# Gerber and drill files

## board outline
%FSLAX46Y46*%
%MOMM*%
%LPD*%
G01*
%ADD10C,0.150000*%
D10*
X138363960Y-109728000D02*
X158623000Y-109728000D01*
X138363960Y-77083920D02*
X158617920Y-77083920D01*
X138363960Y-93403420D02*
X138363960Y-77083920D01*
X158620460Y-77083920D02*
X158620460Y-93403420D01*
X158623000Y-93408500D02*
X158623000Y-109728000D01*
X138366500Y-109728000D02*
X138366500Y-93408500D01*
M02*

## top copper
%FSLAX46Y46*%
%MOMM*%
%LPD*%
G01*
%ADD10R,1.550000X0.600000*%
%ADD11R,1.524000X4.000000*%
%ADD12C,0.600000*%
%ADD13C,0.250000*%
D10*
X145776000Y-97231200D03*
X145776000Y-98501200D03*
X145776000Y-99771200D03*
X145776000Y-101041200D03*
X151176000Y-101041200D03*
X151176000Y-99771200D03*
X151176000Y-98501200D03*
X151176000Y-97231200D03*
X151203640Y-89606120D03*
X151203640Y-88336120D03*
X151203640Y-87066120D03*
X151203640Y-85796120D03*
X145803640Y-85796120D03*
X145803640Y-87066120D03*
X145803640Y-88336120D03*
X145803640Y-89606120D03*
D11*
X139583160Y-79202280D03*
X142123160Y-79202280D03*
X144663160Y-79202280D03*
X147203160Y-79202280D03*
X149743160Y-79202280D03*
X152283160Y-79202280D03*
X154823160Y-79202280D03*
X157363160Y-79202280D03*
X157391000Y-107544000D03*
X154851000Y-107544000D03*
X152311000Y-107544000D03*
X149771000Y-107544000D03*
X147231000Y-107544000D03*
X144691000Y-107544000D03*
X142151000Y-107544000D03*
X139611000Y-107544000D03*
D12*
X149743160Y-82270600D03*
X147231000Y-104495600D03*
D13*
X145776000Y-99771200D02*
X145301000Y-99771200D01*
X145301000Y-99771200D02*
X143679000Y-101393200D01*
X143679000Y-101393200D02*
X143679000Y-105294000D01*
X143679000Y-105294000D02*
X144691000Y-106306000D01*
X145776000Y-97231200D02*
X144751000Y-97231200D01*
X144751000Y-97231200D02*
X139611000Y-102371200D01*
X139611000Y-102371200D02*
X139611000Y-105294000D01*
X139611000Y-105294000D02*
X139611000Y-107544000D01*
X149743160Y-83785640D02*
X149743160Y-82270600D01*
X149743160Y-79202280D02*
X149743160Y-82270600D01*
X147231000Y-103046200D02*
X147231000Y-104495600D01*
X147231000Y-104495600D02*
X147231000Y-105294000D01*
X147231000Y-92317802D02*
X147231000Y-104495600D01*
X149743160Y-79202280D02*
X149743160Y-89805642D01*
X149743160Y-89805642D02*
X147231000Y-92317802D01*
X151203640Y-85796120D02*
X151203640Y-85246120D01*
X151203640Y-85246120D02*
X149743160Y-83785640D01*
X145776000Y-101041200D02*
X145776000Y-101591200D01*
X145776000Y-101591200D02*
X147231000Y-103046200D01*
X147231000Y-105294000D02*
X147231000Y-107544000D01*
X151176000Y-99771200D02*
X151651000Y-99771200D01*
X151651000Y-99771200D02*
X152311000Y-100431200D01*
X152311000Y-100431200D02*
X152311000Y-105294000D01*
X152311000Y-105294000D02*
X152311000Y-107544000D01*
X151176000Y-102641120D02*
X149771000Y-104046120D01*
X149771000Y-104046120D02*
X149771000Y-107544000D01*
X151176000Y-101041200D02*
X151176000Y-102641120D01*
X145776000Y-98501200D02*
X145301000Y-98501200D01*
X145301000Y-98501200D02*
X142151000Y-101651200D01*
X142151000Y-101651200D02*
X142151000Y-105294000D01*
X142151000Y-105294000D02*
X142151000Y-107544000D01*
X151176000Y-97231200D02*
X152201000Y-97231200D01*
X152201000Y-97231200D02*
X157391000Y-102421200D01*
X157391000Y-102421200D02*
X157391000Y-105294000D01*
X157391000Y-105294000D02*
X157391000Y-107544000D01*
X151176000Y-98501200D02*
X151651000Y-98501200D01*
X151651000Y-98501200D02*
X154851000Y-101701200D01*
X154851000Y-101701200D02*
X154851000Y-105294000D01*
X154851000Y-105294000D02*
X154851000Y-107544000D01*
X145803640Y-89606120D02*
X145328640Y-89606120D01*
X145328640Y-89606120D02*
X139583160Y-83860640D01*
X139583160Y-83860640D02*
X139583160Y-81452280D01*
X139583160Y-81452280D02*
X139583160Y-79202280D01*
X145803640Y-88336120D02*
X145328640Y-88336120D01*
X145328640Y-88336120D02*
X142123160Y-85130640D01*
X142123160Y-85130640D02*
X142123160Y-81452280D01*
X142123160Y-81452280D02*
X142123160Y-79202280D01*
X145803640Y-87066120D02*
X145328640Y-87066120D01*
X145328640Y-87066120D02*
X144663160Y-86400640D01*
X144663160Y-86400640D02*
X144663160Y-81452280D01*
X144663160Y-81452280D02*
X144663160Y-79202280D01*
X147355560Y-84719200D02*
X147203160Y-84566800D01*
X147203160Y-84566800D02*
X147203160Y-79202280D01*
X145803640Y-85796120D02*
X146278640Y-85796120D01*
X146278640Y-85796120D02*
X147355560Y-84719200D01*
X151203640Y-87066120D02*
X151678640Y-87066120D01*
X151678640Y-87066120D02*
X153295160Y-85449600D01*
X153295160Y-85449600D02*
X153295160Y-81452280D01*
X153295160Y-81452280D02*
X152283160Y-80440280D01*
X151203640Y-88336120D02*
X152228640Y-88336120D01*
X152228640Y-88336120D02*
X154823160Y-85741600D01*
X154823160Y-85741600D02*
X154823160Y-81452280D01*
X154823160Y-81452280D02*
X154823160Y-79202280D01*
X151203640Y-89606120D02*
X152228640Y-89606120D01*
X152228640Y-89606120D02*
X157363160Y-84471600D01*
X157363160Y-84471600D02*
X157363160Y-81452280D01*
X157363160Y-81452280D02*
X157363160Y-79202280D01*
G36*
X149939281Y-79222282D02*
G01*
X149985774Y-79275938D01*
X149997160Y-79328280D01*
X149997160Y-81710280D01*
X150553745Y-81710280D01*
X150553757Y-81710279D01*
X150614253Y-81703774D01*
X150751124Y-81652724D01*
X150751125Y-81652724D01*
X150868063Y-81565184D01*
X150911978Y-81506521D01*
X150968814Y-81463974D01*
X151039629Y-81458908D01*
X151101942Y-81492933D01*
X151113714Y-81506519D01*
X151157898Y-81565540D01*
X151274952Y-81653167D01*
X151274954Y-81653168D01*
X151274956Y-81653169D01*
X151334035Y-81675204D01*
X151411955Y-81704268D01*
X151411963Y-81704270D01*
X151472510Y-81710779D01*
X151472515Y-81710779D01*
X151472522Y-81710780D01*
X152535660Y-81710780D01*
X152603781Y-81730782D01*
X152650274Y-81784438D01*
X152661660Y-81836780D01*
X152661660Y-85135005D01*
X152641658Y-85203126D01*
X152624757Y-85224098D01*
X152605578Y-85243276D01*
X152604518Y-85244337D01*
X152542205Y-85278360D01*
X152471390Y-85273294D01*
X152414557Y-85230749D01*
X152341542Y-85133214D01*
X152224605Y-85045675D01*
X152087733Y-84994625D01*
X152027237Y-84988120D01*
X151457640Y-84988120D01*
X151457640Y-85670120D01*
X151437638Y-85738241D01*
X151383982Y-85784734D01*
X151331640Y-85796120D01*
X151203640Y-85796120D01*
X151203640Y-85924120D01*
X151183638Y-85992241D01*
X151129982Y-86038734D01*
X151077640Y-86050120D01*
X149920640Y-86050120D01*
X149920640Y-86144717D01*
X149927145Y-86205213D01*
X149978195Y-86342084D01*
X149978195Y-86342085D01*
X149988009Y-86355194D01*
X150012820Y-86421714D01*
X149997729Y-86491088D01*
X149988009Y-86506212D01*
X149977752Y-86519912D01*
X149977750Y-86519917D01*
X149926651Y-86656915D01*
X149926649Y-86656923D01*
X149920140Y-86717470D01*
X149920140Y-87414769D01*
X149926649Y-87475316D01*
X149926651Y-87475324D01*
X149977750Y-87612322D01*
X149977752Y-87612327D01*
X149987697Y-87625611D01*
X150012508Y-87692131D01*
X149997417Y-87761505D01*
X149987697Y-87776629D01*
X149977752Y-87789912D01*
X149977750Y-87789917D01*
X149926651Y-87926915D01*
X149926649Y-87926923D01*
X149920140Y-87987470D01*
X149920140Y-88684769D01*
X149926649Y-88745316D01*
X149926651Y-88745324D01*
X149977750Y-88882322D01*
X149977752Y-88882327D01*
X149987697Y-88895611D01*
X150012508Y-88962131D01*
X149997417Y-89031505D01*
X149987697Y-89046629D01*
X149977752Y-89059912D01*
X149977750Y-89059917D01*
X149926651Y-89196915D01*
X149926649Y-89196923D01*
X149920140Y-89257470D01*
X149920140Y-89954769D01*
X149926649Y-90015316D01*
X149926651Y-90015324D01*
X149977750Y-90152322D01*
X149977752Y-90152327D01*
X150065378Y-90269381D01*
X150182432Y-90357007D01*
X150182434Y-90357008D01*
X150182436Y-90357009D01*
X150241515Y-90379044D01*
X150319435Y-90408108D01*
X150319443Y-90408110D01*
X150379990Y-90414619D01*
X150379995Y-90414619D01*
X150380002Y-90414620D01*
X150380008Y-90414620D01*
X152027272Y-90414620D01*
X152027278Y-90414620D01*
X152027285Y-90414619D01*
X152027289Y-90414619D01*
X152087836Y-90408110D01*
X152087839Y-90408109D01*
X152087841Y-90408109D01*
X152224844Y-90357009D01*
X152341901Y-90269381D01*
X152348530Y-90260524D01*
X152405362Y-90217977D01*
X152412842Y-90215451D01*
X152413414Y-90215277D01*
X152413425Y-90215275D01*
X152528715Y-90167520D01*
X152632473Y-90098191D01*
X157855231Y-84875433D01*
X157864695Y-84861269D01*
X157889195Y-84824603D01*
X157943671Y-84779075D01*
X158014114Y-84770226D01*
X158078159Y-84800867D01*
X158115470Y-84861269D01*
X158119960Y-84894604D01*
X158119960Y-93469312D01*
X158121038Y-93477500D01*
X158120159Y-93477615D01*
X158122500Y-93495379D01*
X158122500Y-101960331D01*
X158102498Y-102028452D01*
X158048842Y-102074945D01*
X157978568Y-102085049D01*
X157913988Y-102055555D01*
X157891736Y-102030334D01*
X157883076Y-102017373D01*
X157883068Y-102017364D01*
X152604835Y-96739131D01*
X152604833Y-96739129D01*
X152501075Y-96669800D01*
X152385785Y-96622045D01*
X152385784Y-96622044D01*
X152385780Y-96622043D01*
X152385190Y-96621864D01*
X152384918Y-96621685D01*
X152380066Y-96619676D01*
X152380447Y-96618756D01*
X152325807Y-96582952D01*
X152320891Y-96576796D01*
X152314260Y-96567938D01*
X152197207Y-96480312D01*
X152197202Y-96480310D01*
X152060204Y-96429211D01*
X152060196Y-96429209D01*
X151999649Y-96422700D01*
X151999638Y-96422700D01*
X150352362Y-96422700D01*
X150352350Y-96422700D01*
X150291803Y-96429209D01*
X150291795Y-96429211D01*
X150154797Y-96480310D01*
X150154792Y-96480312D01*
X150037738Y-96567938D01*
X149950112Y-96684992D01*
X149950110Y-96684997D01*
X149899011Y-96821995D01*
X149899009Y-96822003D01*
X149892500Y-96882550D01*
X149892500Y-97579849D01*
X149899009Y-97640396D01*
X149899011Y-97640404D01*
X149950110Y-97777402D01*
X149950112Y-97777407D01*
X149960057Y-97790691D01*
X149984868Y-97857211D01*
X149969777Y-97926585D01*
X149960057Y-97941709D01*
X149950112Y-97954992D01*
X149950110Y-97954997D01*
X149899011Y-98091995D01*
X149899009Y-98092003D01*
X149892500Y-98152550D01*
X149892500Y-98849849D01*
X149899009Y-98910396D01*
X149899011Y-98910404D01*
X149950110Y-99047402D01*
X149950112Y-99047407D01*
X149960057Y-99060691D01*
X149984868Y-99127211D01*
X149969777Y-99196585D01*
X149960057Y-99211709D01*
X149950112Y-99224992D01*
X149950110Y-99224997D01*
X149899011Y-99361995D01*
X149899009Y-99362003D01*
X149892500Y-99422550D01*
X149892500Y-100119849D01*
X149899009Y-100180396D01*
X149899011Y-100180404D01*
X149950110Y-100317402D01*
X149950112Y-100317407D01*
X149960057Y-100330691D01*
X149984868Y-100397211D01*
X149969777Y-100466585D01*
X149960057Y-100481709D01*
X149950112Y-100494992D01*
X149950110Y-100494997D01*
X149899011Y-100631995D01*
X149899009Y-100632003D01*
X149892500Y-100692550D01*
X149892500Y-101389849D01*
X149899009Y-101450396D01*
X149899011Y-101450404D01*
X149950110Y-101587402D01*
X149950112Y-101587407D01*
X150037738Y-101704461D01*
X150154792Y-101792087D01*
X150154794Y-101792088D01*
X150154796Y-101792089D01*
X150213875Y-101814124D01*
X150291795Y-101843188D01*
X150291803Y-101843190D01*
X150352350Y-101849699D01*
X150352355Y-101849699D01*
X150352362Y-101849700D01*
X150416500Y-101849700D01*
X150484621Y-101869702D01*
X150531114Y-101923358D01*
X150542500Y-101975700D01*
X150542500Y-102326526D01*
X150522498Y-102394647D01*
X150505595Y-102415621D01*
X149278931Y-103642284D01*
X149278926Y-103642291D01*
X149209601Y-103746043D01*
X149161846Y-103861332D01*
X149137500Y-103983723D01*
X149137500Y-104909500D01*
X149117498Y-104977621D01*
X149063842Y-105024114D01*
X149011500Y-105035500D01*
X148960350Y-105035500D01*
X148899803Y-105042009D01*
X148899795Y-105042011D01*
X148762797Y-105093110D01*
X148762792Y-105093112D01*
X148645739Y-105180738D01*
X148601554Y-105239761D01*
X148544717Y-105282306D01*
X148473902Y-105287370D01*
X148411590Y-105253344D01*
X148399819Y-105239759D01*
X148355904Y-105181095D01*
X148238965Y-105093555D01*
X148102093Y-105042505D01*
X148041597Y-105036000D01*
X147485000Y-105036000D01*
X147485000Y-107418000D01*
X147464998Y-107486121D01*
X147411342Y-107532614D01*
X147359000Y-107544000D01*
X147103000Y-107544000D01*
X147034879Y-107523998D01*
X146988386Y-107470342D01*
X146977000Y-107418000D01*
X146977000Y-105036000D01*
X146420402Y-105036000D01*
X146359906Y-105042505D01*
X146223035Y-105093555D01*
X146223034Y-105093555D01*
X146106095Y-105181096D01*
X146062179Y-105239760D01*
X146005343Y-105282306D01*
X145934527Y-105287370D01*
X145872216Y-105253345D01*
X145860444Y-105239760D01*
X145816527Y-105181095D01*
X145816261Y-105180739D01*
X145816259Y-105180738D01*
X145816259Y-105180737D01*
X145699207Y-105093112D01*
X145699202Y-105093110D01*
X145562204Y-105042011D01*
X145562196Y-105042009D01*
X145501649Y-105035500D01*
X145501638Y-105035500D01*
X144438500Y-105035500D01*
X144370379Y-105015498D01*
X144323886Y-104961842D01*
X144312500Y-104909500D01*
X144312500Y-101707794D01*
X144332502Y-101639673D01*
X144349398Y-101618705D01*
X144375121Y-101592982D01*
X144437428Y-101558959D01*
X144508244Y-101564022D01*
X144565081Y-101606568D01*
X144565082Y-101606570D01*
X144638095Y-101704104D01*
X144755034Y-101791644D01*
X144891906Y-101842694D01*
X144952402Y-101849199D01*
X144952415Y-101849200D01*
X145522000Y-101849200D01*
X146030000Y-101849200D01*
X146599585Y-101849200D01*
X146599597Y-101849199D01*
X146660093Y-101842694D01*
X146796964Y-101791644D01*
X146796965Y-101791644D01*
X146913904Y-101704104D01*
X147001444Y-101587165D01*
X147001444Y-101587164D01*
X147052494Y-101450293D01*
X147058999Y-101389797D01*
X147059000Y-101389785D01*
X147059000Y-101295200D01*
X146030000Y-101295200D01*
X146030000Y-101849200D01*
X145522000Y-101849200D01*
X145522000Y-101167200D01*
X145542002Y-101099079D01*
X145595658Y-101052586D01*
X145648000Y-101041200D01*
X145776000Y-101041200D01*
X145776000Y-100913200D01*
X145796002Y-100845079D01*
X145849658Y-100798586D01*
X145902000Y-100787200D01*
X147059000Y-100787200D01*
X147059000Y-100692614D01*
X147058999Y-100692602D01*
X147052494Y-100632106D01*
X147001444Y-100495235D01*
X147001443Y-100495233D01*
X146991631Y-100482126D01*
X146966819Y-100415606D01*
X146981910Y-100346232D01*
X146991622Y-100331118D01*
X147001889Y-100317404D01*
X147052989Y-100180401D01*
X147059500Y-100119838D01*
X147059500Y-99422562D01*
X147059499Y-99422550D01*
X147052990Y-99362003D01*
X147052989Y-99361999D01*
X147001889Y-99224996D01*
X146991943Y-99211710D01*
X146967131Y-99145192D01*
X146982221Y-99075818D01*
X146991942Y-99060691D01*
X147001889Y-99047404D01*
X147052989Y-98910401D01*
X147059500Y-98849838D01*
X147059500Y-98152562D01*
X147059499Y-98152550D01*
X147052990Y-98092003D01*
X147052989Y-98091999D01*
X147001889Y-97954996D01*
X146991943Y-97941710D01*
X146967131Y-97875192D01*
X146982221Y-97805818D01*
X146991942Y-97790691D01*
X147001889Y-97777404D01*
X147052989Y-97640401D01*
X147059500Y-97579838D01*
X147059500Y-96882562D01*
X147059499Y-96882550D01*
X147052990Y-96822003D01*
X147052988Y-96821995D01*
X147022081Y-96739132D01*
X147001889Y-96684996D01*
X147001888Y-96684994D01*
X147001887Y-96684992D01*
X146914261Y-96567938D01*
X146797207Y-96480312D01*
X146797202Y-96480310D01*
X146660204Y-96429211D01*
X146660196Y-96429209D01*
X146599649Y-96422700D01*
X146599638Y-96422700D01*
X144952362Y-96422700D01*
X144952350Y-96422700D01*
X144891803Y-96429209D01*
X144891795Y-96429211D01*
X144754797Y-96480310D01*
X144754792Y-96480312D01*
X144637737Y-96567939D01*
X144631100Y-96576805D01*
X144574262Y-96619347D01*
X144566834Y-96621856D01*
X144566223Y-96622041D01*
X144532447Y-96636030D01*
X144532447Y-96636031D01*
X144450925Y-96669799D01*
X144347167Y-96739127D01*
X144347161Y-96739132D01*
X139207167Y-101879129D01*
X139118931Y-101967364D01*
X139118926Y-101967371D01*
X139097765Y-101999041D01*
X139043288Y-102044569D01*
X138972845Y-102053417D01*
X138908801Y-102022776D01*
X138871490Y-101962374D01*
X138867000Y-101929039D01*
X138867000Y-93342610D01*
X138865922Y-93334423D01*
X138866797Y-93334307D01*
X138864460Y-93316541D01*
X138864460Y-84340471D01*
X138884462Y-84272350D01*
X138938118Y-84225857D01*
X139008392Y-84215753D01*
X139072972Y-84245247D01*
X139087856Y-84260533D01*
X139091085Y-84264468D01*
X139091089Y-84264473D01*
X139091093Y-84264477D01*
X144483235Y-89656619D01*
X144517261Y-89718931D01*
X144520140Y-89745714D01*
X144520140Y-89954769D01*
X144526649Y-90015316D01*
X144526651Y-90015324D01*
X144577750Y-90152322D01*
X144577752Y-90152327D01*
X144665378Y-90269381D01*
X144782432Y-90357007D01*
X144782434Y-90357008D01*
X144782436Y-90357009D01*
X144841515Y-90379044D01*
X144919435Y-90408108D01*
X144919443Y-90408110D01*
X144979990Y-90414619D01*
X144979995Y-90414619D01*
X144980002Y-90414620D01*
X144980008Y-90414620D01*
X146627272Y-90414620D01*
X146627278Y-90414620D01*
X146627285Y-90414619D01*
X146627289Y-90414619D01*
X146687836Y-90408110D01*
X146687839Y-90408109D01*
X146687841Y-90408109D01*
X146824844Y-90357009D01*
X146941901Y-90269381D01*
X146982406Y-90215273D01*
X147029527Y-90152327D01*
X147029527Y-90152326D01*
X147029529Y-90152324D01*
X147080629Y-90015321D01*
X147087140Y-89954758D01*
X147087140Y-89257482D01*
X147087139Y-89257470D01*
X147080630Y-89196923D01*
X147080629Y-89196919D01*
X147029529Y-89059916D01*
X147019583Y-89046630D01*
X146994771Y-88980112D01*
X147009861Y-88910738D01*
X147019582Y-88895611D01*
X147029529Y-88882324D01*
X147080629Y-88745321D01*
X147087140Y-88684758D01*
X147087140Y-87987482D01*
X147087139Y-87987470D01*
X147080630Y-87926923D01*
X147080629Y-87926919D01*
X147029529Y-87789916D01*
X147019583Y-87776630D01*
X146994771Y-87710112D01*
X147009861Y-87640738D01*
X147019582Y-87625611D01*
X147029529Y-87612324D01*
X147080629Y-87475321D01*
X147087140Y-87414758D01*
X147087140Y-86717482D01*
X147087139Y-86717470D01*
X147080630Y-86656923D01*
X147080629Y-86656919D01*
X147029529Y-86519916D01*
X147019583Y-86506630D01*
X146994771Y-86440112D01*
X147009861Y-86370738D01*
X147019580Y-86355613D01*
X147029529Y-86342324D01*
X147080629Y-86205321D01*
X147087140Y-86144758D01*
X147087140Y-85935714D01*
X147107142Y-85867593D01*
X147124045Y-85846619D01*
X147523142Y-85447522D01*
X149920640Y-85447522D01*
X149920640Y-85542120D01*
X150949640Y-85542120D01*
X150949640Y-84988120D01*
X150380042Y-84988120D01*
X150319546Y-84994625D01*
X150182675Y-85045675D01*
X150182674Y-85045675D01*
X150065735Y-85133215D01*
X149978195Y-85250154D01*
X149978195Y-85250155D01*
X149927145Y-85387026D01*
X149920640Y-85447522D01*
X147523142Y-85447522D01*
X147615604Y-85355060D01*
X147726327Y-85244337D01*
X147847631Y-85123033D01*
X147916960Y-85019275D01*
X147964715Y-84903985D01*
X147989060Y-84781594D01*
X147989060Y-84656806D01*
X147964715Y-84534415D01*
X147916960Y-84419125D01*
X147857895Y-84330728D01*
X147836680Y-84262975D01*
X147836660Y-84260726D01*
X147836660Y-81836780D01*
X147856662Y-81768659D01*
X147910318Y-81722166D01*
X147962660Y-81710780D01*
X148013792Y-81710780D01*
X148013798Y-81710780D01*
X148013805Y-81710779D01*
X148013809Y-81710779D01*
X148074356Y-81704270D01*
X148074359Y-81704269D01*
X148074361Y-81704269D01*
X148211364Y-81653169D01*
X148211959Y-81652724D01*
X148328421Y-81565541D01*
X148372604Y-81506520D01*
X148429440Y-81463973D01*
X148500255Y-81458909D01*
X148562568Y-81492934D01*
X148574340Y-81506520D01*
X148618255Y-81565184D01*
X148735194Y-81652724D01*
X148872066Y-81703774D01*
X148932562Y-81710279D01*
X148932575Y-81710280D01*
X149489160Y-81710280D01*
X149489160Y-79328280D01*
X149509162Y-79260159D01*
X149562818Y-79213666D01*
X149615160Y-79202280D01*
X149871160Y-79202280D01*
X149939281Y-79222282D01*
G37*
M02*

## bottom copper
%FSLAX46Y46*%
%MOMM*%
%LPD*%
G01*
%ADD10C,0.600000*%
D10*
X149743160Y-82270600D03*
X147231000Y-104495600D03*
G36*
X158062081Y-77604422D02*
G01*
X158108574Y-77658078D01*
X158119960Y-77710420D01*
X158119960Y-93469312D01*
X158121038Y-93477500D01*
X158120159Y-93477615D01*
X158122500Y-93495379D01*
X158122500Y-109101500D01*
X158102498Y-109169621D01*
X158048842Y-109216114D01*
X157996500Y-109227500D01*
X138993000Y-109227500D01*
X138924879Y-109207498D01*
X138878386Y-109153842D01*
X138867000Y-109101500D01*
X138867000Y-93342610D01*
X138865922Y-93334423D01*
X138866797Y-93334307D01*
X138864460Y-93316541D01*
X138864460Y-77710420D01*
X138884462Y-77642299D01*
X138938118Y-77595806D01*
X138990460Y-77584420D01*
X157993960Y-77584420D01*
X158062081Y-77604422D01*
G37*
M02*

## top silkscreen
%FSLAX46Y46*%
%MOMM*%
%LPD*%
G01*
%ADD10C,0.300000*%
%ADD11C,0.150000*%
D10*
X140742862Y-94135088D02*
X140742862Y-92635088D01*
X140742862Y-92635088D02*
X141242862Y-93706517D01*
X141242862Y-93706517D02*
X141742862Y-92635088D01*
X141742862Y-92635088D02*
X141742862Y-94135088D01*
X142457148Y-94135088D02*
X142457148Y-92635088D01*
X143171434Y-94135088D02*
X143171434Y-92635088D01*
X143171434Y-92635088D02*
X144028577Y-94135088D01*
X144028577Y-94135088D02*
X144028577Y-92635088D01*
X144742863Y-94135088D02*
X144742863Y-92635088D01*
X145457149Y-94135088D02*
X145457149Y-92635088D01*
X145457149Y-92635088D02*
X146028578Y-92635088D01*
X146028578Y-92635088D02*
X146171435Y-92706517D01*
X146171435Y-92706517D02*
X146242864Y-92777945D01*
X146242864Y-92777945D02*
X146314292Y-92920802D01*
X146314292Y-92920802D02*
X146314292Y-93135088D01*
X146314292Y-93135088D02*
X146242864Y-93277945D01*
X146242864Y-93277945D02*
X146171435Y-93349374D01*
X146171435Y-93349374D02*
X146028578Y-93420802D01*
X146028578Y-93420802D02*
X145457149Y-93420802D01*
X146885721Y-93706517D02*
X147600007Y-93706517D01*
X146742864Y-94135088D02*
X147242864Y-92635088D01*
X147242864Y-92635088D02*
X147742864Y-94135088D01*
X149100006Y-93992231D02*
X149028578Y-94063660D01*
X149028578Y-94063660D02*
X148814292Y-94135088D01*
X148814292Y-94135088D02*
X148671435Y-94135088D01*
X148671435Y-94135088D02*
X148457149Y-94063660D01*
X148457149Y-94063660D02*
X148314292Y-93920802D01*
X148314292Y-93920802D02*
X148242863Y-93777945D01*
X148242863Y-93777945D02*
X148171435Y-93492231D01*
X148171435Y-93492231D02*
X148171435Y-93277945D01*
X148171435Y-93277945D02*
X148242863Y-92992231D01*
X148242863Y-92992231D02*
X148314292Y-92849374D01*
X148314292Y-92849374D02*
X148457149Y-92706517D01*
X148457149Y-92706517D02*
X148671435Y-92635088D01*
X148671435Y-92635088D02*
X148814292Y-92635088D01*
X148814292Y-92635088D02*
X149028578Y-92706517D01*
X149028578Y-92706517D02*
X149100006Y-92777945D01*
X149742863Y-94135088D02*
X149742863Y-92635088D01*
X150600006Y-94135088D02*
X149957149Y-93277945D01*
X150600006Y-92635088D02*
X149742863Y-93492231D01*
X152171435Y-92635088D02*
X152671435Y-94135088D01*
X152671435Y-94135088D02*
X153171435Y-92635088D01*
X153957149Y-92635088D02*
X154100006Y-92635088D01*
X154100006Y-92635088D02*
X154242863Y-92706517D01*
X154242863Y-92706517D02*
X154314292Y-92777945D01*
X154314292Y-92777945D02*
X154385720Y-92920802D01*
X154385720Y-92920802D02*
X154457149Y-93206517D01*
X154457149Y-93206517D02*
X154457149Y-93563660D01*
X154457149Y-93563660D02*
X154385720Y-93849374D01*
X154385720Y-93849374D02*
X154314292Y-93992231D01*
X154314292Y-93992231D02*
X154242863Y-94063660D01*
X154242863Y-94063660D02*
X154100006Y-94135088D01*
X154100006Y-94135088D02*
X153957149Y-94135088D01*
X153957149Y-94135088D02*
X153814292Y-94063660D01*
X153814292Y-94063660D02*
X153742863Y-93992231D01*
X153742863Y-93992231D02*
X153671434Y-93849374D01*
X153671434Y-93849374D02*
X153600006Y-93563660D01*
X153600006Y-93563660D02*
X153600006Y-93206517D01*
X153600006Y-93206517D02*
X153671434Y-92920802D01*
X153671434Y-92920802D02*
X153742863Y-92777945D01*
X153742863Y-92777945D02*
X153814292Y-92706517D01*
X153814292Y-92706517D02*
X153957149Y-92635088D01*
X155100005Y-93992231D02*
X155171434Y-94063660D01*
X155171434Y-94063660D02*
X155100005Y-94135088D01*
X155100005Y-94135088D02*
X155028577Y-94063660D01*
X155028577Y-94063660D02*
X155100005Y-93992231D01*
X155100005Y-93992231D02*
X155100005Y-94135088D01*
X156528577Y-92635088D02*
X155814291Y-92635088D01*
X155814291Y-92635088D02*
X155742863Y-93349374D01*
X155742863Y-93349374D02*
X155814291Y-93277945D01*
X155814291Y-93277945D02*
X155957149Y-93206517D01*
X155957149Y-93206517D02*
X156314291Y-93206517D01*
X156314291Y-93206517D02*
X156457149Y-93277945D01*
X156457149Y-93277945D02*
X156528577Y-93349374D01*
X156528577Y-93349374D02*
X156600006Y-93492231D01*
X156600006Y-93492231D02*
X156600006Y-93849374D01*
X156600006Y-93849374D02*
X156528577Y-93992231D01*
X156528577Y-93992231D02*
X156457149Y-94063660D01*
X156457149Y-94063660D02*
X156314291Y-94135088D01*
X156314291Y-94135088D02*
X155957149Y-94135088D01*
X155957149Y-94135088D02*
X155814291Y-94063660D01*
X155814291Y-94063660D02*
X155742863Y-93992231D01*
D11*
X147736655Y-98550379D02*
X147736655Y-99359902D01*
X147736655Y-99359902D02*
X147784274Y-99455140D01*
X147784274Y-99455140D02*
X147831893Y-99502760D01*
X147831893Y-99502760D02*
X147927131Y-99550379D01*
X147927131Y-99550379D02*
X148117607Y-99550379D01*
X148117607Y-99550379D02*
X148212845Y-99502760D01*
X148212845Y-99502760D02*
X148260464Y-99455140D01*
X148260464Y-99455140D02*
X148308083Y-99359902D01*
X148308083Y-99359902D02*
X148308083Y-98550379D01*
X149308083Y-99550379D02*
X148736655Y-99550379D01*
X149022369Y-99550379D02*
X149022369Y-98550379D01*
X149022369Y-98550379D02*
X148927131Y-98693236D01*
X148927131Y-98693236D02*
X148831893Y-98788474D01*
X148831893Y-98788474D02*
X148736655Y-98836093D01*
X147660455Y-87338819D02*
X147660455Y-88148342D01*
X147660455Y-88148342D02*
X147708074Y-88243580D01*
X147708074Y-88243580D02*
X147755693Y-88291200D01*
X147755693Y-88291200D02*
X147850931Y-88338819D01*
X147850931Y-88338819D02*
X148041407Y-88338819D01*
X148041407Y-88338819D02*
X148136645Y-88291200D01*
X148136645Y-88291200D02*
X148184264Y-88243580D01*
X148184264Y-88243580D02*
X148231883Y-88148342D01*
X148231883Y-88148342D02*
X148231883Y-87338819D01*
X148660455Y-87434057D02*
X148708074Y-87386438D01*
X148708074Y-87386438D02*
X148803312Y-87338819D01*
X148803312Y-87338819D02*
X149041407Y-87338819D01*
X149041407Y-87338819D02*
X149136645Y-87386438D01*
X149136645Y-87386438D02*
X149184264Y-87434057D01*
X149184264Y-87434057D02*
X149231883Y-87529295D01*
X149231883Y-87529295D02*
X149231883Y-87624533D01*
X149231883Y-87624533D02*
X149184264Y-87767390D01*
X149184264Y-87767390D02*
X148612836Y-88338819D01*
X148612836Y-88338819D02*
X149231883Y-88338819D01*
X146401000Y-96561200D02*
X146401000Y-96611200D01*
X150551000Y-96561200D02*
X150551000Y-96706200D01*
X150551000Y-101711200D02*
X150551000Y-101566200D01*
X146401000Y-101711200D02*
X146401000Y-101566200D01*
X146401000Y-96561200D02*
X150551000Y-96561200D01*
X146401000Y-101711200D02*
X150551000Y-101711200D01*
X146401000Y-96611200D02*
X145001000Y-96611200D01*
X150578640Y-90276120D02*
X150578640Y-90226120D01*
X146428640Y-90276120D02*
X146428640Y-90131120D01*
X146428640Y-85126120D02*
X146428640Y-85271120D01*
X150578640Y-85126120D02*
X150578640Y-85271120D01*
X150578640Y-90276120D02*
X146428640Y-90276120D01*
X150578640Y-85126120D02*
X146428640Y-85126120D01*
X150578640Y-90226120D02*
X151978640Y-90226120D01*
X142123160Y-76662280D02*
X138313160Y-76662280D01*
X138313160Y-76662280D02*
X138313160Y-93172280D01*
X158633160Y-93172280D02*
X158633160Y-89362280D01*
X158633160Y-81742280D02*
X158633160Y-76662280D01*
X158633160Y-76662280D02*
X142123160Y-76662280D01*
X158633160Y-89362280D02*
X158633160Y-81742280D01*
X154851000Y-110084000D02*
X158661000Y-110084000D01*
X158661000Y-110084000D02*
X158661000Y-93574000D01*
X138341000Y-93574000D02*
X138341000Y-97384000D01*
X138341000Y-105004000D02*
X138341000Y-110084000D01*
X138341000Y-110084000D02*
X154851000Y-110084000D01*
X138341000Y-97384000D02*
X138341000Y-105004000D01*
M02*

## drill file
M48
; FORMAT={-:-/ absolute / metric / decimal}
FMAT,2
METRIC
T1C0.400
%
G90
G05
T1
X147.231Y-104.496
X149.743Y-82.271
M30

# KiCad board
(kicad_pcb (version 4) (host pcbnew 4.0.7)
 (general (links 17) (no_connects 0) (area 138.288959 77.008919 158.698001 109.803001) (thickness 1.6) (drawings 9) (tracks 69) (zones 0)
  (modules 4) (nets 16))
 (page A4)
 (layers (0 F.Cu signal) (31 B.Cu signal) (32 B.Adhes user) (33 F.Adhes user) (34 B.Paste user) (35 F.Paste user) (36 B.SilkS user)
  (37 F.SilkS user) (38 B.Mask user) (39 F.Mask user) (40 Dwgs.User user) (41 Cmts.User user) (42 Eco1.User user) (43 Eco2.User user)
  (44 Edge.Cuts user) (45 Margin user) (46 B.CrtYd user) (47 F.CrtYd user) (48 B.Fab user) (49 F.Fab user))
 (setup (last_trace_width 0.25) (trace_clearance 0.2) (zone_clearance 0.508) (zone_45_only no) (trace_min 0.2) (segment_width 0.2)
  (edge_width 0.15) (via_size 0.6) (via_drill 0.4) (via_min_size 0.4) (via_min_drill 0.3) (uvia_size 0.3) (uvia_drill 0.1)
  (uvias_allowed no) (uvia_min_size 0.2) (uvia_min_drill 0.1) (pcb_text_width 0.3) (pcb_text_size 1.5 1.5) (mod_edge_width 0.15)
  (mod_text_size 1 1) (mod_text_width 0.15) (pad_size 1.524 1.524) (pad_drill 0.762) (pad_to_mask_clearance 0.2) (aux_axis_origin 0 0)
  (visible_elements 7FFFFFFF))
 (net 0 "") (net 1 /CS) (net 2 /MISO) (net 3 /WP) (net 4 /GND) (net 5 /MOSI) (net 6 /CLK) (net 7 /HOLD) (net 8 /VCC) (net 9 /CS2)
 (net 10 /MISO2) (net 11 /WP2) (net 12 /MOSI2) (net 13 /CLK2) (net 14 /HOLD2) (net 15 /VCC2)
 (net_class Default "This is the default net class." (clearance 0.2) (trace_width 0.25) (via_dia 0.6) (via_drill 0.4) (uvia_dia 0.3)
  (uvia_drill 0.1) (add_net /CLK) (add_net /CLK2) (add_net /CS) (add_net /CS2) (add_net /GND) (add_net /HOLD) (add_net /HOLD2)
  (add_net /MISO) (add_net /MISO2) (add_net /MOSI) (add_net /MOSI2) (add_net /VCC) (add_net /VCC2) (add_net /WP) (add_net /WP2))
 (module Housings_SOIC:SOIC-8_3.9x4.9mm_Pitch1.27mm (layer F.Cu) (at 148.476 99.1362)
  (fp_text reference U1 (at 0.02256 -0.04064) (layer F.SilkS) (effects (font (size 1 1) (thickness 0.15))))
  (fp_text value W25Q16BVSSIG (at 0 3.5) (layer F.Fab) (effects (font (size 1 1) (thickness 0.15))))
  (fp_line (start -2.075 -2.575) (end -2.075 -2.525) (layer F.SilkS) (width 0.15))
  (fp_line (start 2.075 -2.575) (end 2.075 -2.43) (layer F.SilkS) (width 0.15))
  (fp_line (start 2.075 2.575) (end 2.075 2.43) (layer F.SilkS) (width 0.15))
  (fp_line (start -2.075 2.575) (end -2.075 2.43) (layer F.SilkS) (width 0.15))
  (fp_line (start -2.075 -2.575) (end 2.075 -2.575) (layer F.SilkS) (width 0.15))
  (fp_line (start -2.075 2.575) (end 2.075 2.575) (layer F.SilkS) (width 0.15))
  (fp_line (start -2.075 -2.525) (end -3.475 -2.525) (layer F.SilkS) (width 0.15))
  (pad 1 smd rect (at -2.7 -1.905) (size 1.55 0.6) (layers F.Cu F.Paste F.Mask) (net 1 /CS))
  (pad 2 smd rect (at -2.7 -0.635) (size 1.55 0.6) (layers F.Cu F.Paste F.Mask) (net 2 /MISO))
  (pad 3 smd rect (at -2.7 0.635) (size 1.55 0.6) (layers F.Cu F.Paste F.Mask) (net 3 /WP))
  (pad 4 smd rect (at -2.7 1.905) (size 1.55 0.6) (layers F.Cu F.Paste F.Mask) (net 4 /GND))
  (pad 5 smd rect (at 2.7 1.905) (size 1.55 0.6) (layers F.Cu F.Paste F.Mask) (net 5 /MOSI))
  (pad 6 smd rect (at 2.7 0.635) (size 1.55 0.6) (layers F.Cu F.Paste F.Mask) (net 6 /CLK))
  (pad 7 smd rect (at 2.7 -0.635) (size 1.55 0.6) (layers F.Cu F.Paste F.Mask) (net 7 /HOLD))
  (pad 8 smd rect (at 2.7 -1.905) (size 1.55 0.6) (layers F.Cu F.Paste F.Mask) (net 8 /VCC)))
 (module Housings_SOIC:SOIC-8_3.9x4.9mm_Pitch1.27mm (layer F.Cu) (at 148.50364 87.70112 180)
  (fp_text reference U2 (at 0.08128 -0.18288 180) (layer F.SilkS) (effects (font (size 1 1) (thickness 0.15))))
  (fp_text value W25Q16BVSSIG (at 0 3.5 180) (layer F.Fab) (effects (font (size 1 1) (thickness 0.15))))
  (fp_line (start -2.075 -2.575) (end -2.075 -2.525) (layer F.SilkS) (width 0.15))
  (fp_line (start 2.075 -2.575) (end 2.075 -2.43) (layer F.SilkS) (width 0.15))
  (fp_line (start 2.075 2.575) (end 2.075 2.43) (layer F.SilkS) (width 0.15))
  (fp_line (start -2.075 2.575) (end -2.075 2.43) (layer F.SilkS) (width 0.15))
  (fp_line (start -2.075 -2.575) (end 2.075 -2.575) (layer F.SilkS) (width 0.15))
  (fp_line (start -2.075 2.575) (end 2.075 2.575) (layer F.SilkS) (width 0.15))
  (fp_line (start -2.075 -2.525) (end -3.475 -2.525) (layer F.SilkS) (width 0.15))
  (pad 1 smd rect (at -2.7 -1.905 180) (size 1.55 0.6) (layers F.Cu F.Paste F.Mask) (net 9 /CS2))
  (pad 2 smd rect (at -2.7 -0.635 180) (size 1.55 0.6) (layers F.Cu F.Paste F.Mask) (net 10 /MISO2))
  (pad 3 smd rect (at -2.7 0.635 180) (size 1.55 0.6) (layers F.Cu F.Paste F.Mask) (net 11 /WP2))
  (pad 4 smd rect (at -2.7 1.905 180) (size 1.55 0.6) (layers F.Cu F.Paste F.Mask) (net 4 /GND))
  (pad 5 smd rect (at 2.7 1.905 180) (size 1.55 0.6) (layers F.Cu F.Paste F.Mask) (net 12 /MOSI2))
  (pad 6 smd rect (at 2.7 0.635 180) (size 1.55 0.6) (layers F.Cu F.Paste F.Mask) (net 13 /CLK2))
  (pad 7 smd rect (at 2.7 -0.635 180) (size 1.55 0.6) (layers F.Cu F.Paste F.Mask) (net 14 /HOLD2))
  (pad 8 smd rect (at 2.7 -1.905 180) (size 1.55 0.6) (layers F.Cu F.Paste F.Mask) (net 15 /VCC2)))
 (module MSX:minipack (layer F.Cu) (at 148.47316 81.74228 180)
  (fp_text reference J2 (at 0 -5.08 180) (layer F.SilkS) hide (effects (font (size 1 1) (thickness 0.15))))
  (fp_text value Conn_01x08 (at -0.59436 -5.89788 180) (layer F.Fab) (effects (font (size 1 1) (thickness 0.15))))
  (fp_line (start 6.35 5.08) (end 10.16 5.08) (layer F.SilkS) (width 0.15))
  (fp_line (start 10.16 5.08) (end 10.16 -11.43) (layer F.SilkS) (width 0.15))
  (fp_line (start -10.16 -11.43) (end -10.16 -7.62) (layer F.SilkS) (width 0.15))
  (fp_line (start -10.16 0) (end -10.16 5.08) (layer F.SilkS) (width 0.15))
  (fp_line (start -10.16 5.08) (end 6.35 5.08) (layer F.SilkS) (width 0.15))
  (fp_line (start -10.16 -7.62) (end -10.16 0) (layer F.SilkS) (width 0.15))
  (pad 8 smd rect (at 8.89 2.54 180) (size 1.524 4) (layers F.Cu F.Paste F.Mask) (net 15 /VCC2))
  (pad 7 smd rect (at 6.35 2.54 180) (size 1.524 4) (layers F.Cu F.Paste F.Mask) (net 14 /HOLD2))
  (pad 6 smd rect (at 3.81 2.54 180) (size 1.524 4) (layers F.Cu F.Paste F.Mask) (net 13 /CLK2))
  (pad 5 smd rect (at 1.27 2.54 180) (size 1.524 4) (layers F.Cu F.Paste F.Mask) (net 12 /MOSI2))
  (pad 4 smd rect (at -1.27 2.54 180) (size 1.524 4) (layers F.Cu F.Paste F.Mask) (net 4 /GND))
  (pad 3 smd rect (at -3.81 2.54 180) (size 1.524 4) (layers F.Cu F.Paste F.Mask) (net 11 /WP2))
  (pad 2 smd rect (at -6.35 2.54 180) (size 1.524 4) (layers F.Cu F.Paste F.Mask) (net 10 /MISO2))
  (pad 1 smd rect (at -8.89 2.54 180) (size 1.524 4) (layers F.Cu F.Paste F.Mask) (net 9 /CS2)))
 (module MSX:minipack (layer F.Cu) (at 148.501 105.004)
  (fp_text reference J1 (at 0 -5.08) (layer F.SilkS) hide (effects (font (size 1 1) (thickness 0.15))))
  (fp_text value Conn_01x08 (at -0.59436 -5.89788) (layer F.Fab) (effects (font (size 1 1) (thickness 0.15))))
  (fp_line (start 6.35 5.08) (end 10.16 5.08) (layer F.SilkS) (width 0.15))
  (fp_line (start 10.16 5.08) (end 10.16 -11.43) (layer F.SilkS) (width 0.15))
  (fp_line (start -10.16 -11.43) (end -10.16 -7.62) (layer F.SilkS) (width 0.15))
  (fp_line (start -10.16 0) (end -10.16 5.08) (layer F.SilkS) (width 0.15))
  (fp_line (start -10.16 5.08) (end 6.35 5.08) (layer F.SilkS) (width 0.15))
  (fp_line (start -10.16 -7.62) (end -10.16 0) (layer F.SilkS) (width 0.15))
  (pad 8 smd rect (at 8.89 2.54) (size 1.524 4) (layers F.Cu F.Paste F.Mask) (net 8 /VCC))
  (pad 7 smd rect (at 6.35 2.54) (size 1.524 4) (layers F.Cu F.Paste F.Mask) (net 7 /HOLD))
  (pad 6 smd rect (at 3.81 2.54) (size 1.524 4) (layers F.Cu F.Paste F.Mask) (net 6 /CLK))
  (pad 5 smd rect (at 1.27 2.54) (size 1.524 4) (layers F.Cu F.Paste F.Mask) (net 5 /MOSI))
  (pad 4 smd rect (at -1.27 2.54) (size 1.524 4) (layers F.Cu F.Paste F.Mask) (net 4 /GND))
  (pad 3 smd rect (at -3.81 2.54) (size 1.524 4) (layers F.Cu F.Paste F.Mask) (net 3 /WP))
  (pad 2 smd rect (at -6.35 2.54) (size 1.524 4) (layers F.Cu F.Paste F.Mask) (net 2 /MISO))
  (pad 1 smd rect (at -8.89 2.54) (size 1.524 4) (layers F.Cu F.Paste F.Mask) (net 1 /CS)))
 (gr_line (start 138.36396 109.728) (end 158.623 109.728) (layer Edge.Cuts) (width 0.15))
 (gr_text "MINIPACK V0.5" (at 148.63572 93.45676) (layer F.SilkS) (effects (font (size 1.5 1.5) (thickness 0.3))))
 (gr_line (start 138.36396 77.08392) (end 158.61792 77.08392) (layer Edge.Cuts) (width 0.15))
 (gr_line (start 138.36396 93.40342) (end 138.36396 77.08392) (layer Edge.Cuts) (width 0.15))
 (gr_line (start 158.62046 77.08392) (end 158.62046 93.40342) (layer Edge.Cuts) (width 0.15))
 (gr_line (start 158.623 93.4085) (end 158.623 109.728) (layer Edge.Cuts) (width 0.15))
 (gr_line (start 138.3665 109.728) (end 138.3665 93.4085) (layer Edge.Cuts) (width 0.15))
 (segment (start 145.776 99.7712) (end 145.301 99.7712) (width 0.25) (layer F.Cu) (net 3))
 (segment (start 145.301 99.7712) (end 143.679 101.3932) (width 0.25) (layer F.Cu) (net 3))
 (segment (start 143.679 101.3932) (end 143.679 105.294) (width 0.25) (layer F.Cu) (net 3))
 (segment (start 143.679 105.294) (end 144.691 106.306) (width 0.25) (layer F.Cu) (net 3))
 (segment (start 145.776 97.2312) (end 144.751 97.2312) (width 0.25) (layer F.Cu) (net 1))
 (segment (start 144.751 97.2312) (end 139.611 102.3712) (width 0.25) (layer F.Cu) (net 1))
 (segment (start 139.611 102.3712) (end 139.611 105.294) (width 0.25) (layer F.Cu) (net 1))
 (segment (start 139.611 105.294) (end 139.611 107.544) (width 0.25) (layer F.Cu) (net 1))
 (segment (start 149.74316 83.78564) (end 149.74316 82.2706) (width 0.25) (layer F.Cu) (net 4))
 (segment (start 149.74316 79.20228) (end 149.74316 82.2706) (width 0.25) (layer F.Cu) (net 4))
 (via (at 149.74316 82.2706) (size 0.6) (drill 0.4) (layers F.Cu B.Cu) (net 4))
 (segment (start 147.231 103.0462) (end 147.231 104.4956) (width 0.25) (layer F.Cu) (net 4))
 (segment (start 147.231 104.4956) (end 147.231 105.294) (width 0.25) (layer F.Cu) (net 4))
 (segment (start 147.231 92.317802) (end 147.231 104.4956) (width 0.25) (layer F.Cu) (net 4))
 (segment (start 149.74316 79.20228) (end 149.74316 89.805642) (width 0.25) (layer F.Cu) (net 4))
 (segment (start 149.74316 89.805642) (end 147.231 92.317802) (width 0.25) (layer F.Cu) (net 4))
 (via (at 147.231 104.4956) (size 0.6) (drill 0.4) (layers F.Cu B.Cu) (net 4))
 (segment (start 151.20364 85.79612) (end 151.20364 85.24612) (width 0.25) (layer F.Cu) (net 4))
 (segment (start 151.20364 85.24612) (end 149.74316 83.78564) (width 0.25) (layer F.Cu) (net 4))
 (segment (start 145.776 101.0412) (end 145.776 101.5912) (width 0.25) (layer F.Cu) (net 4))
 (segment (start 145.776 101.5912) (end 147.231 103.0462) (width 0.25) (layer F.Cu) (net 4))
 (segment (start 147.231 105.294) (end 147.231 107.544) (width 0.25) (layer F.Cu) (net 4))
 (segment (start 151.176 99.7712) (end 151.651 99.7712) (width 0.25) (layer F.Cu) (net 6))
 (segment (start 151.651 99.7712) (end 152.311 100.4312) (width 0.25) (layer F.Cu) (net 6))
 (segment (start 152.311 100.4312) (end 152.311 105.294) (width 0.25) (layer F.Cu) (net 6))
 (segment (start 152.311 105.294) (end 152.311 107.544) (width 0.25) (layer F.Cu) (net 6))
 (segment (start 151.176 102.64112) (end 149.771 104.04612) (width 0.25) (layer F.Cu) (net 5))
 (segment (start 149.771 104.04612) (end 149.771 107.544) (width 0.25) (layer F.Cu) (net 5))
 (segment (start 151.176 101.0412) (end 151.176 102.64112) (width 0.25) (layer F.Cu) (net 5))
 (segment (start 145.776 98.5012) (end 145.301 98.5012) (width 0.25) (layer F.Cu) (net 2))
 (segment (start 145.301 98.5012) (end 142.151 101.6512) (width 0.25) (layer F.Cu) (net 2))
 (segment (start 142.151 101.6512) (end 142.151 105.294) (width 0.25) (layer F.Cu) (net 2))
 (segment (start 142.151 105.294) (end 142.151 107.544) (width 0.25) (layer F.Cu) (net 2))
 (segment (start 151.176 97.2312) (end 152.201 97.2312) (width 0.25) (layer F.Cu) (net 8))
 (segment (start 152.201 97.2312) (end 157.391 102.4212) (width 0.25) (layer F.Cu) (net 8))
 (segment (start 157.391 102.4212) (end 157.391 105.294) (width 0.25) (layer F.Cu) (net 8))
 (segment (start 157.391 105.294) (end 157.391 107.544) (width 0.25) (layer F.Cu) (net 8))
 (segment (start 151.176 98.5012) (end 151.651 98.5012) (width 0.25) (layer F.Cu) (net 7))
 (segment (start 151.651 98.5012) (end 154.851 101.7012) (width 0.25) (layer F.Cu) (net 7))
 (segment (start 154.851 101.7012) (end 154.851 105.294) (width 0.25) (layer F.Cu) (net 7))
 (segment (start 154.851 105.294) (end 154.851 107.544) (width 0.25) (layer F.Cu) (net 7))
 (segment (start 145.80364 89.60612) (end 145.32864 89.60612) (width 0.25) (layer F.Cu) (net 15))
 (segment (start 145.32864 89.60612) (end 139.58316 83.86064) (width 0.25) (layer F.Cu) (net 15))
 (segment (start 139.58316 83.86064) (end 139.58316 81.45228) (width 0.25) (layer F.Cu) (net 15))
 (segment (start 139.58316 81.45228) (end 139.58316 79.20228) (width 0.25) (layer F.Cu) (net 15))
 (segment (start 145.80364 88.33612) (end 145.32864 88.33612) (width 0.25) (layer F.Cu) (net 14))
 (segment (start 145.32864 88.33612) (end 142.12316 85.13064) (width 0.25) (layer F.Cu) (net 14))
 (segment (start 142.12316 85.13064) (end 142.12316 81.45228) (width 0.25) (layer F.Cu) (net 14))
 (segment (start 142.12316 81.45228) (end 142.12316 79.20228) (width 0.25) (layer F.Cu) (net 14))
 (segment (start 145.80364 87.06612) (end 145.32864 87.06612) (width 0.25) (layer F.Cu) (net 13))
 (segment (start 145.32864 87.06612) (end 144.66316 86.40064) (width 0.25) (layer F.Cu) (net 13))
 (segment (start 144.66316 86.40064) (end 144.66316 81.45228) (width 0.25) (layer F.Cu) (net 13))
 (segment (start 144.66316 81.45228) (end 144.66316 79.20228) (width 0.25) (layer F.Cu) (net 13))
 (segment (start 147.35556 84.7192) (end 147.20316 84.5668) (width 0.25) (layer F.Cu) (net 12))
 (segment (start 147.20316 84.5668) (end 147.20316 79.20228) (width 0.25) (layer F.Cu) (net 12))
 (segment (start 145.80364 85.79612) (end 146.27864 85.79612) (width 0.25) (layer F.Cu) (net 12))
 (segment (start 146.27864 85.79612) (end 147.35556 84.7192) (width 0.25) (layer F.Cu) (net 12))
 (segment (start 151.20364 87.06612) (end 151.67864 87.06612) (width 0.25) (layer F.Cu) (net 11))
 (segment (start 151.67864 87.06612) (end 153.29516 85.4496) (width 0.25) (layer F.Cu) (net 11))
 (segment (start 153.29516 85.4496) (end 153.29516 81.45228) (width 0.25) (layer F.Cu) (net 11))
 (segment (start 153.29516 81.45228) (end 152.28316 80.44028) (width 0.25) (layer F.Cu) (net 11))
 (segment (start 151.20364 88.33612) (end 152.22864 88.33612) (width 0.25) (layer F.Cu) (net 10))
 (segment (start 152.22864 88.33612) (end 154.82316 85.7416) (width 0.25) (layer F.Cu) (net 10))
 (segment (start 154.82316 85.7416) (end 154.82316 81.45228) (width 0.25) (layer F.Cu) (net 10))
 (segment (start 154.82316 81.45228) (end 154.82316 79.20228) (width 0.25) (layer F.Cu) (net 10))
 (segment (start 151.20364 89.60612) (end 152.22864 89.60612) (width 0.25) (layer F.Cu) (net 9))
 (segment (start 152.22864 89.60612) (end 157.36316 84.4716) (width 0.25) (layer F.Cu) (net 9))
 (segment (start 157.36316 84.4716) (end 157.36316 81.45228) (width 0.25) (layer F.Cu) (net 9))
 (segment (start 157.36316 81.45228) (end 157.36316 79.20228) (width 0.25) (layer F.Cu) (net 9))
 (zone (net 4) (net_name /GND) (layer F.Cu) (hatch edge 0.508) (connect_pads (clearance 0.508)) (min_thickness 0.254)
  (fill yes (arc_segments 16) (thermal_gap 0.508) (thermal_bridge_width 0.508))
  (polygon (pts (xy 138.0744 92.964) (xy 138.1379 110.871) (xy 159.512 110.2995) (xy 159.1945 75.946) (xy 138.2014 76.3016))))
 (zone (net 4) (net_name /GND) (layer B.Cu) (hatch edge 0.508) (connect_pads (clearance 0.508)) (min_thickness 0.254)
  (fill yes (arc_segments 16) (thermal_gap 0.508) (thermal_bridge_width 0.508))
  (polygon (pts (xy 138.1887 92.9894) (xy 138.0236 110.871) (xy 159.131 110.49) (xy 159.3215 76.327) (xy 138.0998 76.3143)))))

